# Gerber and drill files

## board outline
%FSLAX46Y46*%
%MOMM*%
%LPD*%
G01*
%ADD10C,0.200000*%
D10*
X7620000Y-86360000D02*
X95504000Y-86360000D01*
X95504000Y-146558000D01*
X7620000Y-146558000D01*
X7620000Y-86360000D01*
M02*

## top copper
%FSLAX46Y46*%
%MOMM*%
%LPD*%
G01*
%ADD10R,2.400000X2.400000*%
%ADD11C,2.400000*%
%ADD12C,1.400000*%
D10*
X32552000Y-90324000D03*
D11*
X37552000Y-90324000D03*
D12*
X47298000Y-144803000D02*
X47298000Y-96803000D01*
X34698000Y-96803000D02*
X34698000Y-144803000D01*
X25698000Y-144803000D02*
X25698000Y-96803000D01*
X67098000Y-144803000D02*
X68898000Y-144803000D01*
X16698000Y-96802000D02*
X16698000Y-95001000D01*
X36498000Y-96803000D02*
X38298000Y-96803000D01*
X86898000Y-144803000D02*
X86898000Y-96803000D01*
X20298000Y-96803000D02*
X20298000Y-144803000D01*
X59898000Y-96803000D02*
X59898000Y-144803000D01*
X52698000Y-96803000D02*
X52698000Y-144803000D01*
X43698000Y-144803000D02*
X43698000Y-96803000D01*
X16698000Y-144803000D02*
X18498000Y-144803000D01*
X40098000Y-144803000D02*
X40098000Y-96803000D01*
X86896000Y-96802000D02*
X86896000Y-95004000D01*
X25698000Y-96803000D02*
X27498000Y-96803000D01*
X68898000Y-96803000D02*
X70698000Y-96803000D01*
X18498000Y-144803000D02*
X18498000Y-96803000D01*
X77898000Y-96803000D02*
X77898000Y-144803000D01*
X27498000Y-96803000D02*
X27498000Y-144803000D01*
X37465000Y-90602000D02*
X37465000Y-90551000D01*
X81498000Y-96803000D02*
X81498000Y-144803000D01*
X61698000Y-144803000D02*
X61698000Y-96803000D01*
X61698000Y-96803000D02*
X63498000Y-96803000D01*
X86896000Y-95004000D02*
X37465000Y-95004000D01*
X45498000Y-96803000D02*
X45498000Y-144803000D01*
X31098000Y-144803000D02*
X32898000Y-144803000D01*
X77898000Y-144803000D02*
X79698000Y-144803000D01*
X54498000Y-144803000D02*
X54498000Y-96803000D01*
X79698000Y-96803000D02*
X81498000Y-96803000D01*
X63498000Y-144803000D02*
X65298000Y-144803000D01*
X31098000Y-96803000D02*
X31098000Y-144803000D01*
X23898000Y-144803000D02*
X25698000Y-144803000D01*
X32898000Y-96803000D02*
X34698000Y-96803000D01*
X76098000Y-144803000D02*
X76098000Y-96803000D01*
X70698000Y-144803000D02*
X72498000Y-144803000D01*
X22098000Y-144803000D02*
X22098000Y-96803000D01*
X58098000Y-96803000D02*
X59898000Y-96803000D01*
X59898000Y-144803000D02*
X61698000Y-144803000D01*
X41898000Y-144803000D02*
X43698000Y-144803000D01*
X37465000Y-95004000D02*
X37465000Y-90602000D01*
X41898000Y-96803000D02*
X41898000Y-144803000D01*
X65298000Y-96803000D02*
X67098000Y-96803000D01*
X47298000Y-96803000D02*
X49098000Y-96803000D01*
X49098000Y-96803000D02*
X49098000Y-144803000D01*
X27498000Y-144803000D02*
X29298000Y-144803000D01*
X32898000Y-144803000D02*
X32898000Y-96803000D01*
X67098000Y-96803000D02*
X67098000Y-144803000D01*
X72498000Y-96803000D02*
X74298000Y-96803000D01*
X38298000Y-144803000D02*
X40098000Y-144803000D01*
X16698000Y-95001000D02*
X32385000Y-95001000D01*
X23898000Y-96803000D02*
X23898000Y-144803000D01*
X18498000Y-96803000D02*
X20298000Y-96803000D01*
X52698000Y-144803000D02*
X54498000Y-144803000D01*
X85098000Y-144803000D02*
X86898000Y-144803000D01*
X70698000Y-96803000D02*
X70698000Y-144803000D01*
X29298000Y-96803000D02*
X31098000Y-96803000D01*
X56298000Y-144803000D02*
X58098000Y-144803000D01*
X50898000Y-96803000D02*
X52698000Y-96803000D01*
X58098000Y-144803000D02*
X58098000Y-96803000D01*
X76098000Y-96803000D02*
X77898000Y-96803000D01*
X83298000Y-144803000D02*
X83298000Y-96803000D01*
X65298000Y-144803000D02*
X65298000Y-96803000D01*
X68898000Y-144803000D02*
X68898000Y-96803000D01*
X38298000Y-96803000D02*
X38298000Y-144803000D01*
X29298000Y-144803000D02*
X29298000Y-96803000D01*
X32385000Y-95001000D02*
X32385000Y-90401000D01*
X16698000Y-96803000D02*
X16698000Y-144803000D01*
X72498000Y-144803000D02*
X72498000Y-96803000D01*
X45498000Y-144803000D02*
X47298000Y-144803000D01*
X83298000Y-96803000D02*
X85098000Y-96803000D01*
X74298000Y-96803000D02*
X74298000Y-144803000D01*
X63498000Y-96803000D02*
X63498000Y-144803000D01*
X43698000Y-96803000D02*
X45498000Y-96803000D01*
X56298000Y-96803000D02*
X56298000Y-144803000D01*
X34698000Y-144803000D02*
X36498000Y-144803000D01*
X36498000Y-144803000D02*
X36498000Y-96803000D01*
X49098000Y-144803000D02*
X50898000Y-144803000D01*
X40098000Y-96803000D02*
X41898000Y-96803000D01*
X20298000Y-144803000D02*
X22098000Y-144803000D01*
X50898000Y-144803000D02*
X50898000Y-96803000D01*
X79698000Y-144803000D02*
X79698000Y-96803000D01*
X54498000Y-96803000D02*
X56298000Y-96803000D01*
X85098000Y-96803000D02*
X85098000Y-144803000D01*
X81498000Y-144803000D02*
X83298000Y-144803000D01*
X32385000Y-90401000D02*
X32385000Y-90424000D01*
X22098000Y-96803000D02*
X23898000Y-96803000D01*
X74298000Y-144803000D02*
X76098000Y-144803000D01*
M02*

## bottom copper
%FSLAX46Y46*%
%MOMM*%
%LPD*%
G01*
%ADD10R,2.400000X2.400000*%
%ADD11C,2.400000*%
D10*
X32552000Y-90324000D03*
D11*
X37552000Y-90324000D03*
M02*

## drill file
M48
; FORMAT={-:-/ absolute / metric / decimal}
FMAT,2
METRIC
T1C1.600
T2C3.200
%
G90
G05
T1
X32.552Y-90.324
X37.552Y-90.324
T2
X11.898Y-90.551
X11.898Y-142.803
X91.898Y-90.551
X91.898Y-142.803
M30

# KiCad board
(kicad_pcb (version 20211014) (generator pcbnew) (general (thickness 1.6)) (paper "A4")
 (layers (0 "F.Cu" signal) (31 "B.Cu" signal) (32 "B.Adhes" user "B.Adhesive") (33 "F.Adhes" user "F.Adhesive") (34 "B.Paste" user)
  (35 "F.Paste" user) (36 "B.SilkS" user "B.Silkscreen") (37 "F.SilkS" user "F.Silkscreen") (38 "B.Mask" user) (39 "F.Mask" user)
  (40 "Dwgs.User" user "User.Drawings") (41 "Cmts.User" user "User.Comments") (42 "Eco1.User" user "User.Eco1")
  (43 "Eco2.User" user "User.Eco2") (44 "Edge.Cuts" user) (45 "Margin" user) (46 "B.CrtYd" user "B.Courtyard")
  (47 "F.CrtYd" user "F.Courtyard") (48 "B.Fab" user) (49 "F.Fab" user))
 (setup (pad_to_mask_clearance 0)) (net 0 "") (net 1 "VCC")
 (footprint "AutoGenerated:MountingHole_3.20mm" (layer "F.Cu") (at 91.898 142.803)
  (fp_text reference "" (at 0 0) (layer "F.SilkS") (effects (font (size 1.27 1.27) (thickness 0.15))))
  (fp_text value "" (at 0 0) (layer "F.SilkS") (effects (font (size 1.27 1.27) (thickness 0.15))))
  (pad "" np_thru_hole circle locked (at 0 0) (size 3.2 3.2) (drill 3.2) (layers *.Cu *.Mask)))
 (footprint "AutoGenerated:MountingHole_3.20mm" (layer "F.Cu") (at 11.898 90.551)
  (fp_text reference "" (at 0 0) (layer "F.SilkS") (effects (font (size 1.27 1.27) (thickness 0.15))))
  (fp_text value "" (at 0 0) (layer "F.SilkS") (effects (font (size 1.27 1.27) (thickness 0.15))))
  (pad "" np_thru_hole circle locked (at 0 0) (size 3.2 3.2) (drill 3.2) (layers *.Cu *.Mask)))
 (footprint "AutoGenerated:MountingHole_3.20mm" (layer "F.Cu") (at 91.898 90.551)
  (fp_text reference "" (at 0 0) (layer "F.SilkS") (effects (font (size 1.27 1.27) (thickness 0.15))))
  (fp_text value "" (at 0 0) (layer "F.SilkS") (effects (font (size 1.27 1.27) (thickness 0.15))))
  (pad "" np_thru_hole circle locked (at 0 0) (size 3.2 3.2) (drill 3.2) (layers *.Cu *.Mask)))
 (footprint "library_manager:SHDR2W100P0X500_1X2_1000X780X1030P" (layer "F.Cu") (at 32.552 90.324)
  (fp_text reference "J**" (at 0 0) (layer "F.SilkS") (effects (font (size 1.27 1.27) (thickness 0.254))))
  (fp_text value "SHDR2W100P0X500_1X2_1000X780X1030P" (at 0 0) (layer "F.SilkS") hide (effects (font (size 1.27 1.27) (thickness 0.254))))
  (pad "1" thru_hole rect locked (at 0 0) (size 2.4 2.4) (drill 1.6) (layers *.Cu *.Mask))
  (pad "2" thru_hole circle locked (at 5 0) (size 2.4 2.4) (drill 1.6) (layers *.Cu *.Mask)))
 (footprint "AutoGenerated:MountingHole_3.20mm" (layer "F.Cu") (at 11.898 142.803)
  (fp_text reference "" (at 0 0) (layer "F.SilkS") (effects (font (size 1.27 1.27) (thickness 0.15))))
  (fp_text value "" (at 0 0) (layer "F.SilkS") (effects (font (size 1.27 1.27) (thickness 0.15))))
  (pad "" np_thru_hole circle locked (at 0 0) (size 3.2 3.2) (drill 3.2) (layers *.Cu *.Mask)))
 (gr_rect (start 7.62 86.36) (end 95.504 146.558) (layer "Edge.Cuts") (width 0.2) (fill none))
 (segment (start 47.298 144.803) (end 47.298 96.803) (width 1.4) (layer "F.Cu") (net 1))
 (segment (start 34.698 96.803) (end 34.698 144.803) (width 1.4) (layer "F.Cu") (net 1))
 (segment (start 25.698 144.803) (end 25.698 96.803) (width 1.4) (layer "F.Cu") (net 1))
 (segment (start 67.098 144.803) (end 68.898 144.803) (width 1.4) (layer "F.Cu") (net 1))
 (segment (start 16.698 96.802) (end 16.698 95.001) (width 1.4) (layer "F.Cu") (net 1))
 (segment (start 36.498 96.803) (end 38.298 96.803) (width 1.4) (layer "F.Cu") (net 1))
 (segment (start 86.898 144.803) (end 86.898 96.803) (width 1.4) (layer "F.Cu") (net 1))
 (segment (start 20.298 96.803) (end 20.298 144.803) (width 1.4) (layer "F.Cu") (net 1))
 (segment (start 59.898 96.803) (end 59.898 144.803) (width 1.4) (layer "F.Cu") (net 1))
 (segment (start 52.698 96.803) (end 52.698 144.803) (width 1.4) (layer "F.Cu") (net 1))
 (segment (start 43.698 144.803) (end 43.698 96.803) (width 1.4) (layer "F.Cu") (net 1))
 (segment (start 16.698 144.803) (end 18.498 144.803) (width 1.4) (layer "F.Cu") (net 1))
 (segment (start 40.098 144.803) (end 40.098 96.803) (width 1.4) (layer "F.Cu") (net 1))
 (segment (start 86.896 96.802) (end 86.896 95.004) (width 1.4) (layer "F.Cu") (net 1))
 (segment (start 25.698 96.803) (end 27.498 96.803) (width 1.4) (layer "F.Cu") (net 1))
 (segment (start 68.898 96.803) (end 70.698 96.803) (width 1.4) (layer "F.Cu") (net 1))
 (segment (start 18.498 144.803) (end 18.498 96.803) (width 1.4) (layer "F.Cu") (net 1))
 (segment (start 77.898 96.803) (end 77.898 144.803) (width 1.4) (layer "F.Cu") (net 1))
 (segment (start 27.498 96.803) (end 27.498 144.803) (width 1.4) (layer "F.Cu") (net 1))
 (segment (start 37.465 90.602) (end 37.465 90.551) (width 1.4) (layer "F.Cu") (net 1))
 (segment (start 81.498 96.803) (end 81.498 144.803) (width 1.4) (layer "F.Cu") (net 1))
 (segment (start 61.698 144.803) (end 61.698 96.803) (width 1.4) (layer "F.Cu") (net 1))
 (segment (start 61.698 96.803) (end 63.498 96.803) (width 1.4) (layer "F.Cu") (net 1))
 (segment (start 86.896 95.004) (end 37.465 95.004) (width 1.4) (layer "F.Cu") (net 1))
 (segment (start 45.498 96.803) (end 45.498 144.803) (width 1.4) (layer "F.Cu") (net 1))
 (segment (start 31.098 144.803) (end 32.898 144.803) (width 1.4) (layer "F.Cu") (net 1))
 (segment (start 77.898 144.803) (end 79.698 144.803) (width 1.4) (layer "F.Cu") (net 1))
 (segment (start 54.498 144.803) (end 54.498 96.803) (width 1.4) (layer "F.Cu") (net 1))
 (segment (start 79.698 96.803) (end 81.498 96.803) (width 1.4) (layer "F.Cu") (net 1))
 (segment (start 63.498 144.803) (end 65.298 144.803) (width 1.4) (layer "F.Cu") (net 1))
 (segment (start 31.098 96.803) (end 31.098 144.803) (width 1.4) (layer "F.Cu") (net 1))
 (segment (start 23.898 144.803) (end 25.698 144.803) (width 1.4) (layer "F.Cu") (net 1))
 (segment (start 32.898 96.803) (end 34.698 96.803) (width 1.4) (layer "F.Cu") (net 1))
 (segment (start 76.098 144.803) (end 76.098 96.803) (width 1.4) (layer "F.Cu") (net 1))
 (segment (start 70.698 144.803) (end 72.498 144.803) (width 1.4) (layer "F.Cu") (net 1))
 (segment (start 22.098 144.803) (end 22.098 96.803) (width 1.4) (layer "F.Cu") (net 1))
 (segment (start 58.098 96.803) (end 59.898 96.803) (width 1.4) (layer "F.Cu") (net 1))
 (segment (start 59.898 144.803) (end 61.698 144.803) (width 1.4) (layer "F.Cu") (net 1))
 (segment (start 41.898 144.803) (end 43.698 144.803) (width 1.4) (layer "F.Cu") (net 1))
 (segment (start 37.465 95.004) (end 37.465 90.602) (width 1.4) (layer "F.Cu") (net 1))
 (segment (start 41.898 96.803) (end 41.898 144.803) (width 1.4) (layer "F.Cu") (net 1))
 (segment (start 65.298 96.803) (end 67.098 96.803) (width 1.4) (layer "F.Cu") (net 1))
 (segment (start 47.298 96.803) (end 49.098 96.803) (width 1.4) (layer "F.Cu") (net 1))
 (segment (start 49.098 96.803) (end 49.098 144.803) (width 1.4) (layer "F.Cu") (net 1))
 (segment (start 27.498 144.803) (end 29.298 144.803) (width 1.4) (layer "F.Cu") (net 1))
 (segment (start 32.898 144.803) (end 32.898 96.803) (width 1.4) (layer "F.Cu") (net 1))
 (segment (start 67.098 96.803) (end 67.098 144.803) (width 1.4) (layer "F.Cu") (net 1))
 (segment (start 72.498 96.803) (end 74.298 96.803) (width 1.4) (layer "F.Cu") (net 1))
 (segment (start 38.298 144.803) (end 40.098 144.803) (width 1.4) (layer "F.Cu") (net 1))
 (segment (start 16.698 95.001) (end 32.385 95.001) (width 1.4) (layer "F.Cu") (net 1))
 (segment (start 23.898 96.803) (end 23.898 144.803) (width 1.4) (layer "F.Cu") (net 1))
 (segment (start 18.498 96.803) (end 20.298 96.803) (width 1.4) (layer "F.Cu") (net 1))
 (segment (start 52.698 144.803) (end 54.498 144.803) (width 1.4) (layer "F.Cu") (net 1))
 (segment (start 85.098 144.803) (end 86.898 144.803) (width 1.4) (layer "F.Cu") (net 1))
 (segment (start 70.698 96.803) (end 70.698 144.803) (width 1.4) (layer "F.Cu") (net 1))
 (segment (start 29.298 96.803) (end 31.098 96.803) (width 1.4) (layer "F.Cu") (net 1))
 (segment (start 56.298 144.803) (end 58.098 144.803) (width 1.4) (layer "F.Cu") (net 1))
 (segment (start 50.898 96.803) (end 52.698 96.803) (width 1.4) (layer "F.Cu") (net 1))
 (segment (start 58.098 144.803) (end 58.098 96.803) (width 1.4) (layer "F.Cu") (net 1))
 (segment (start 76.098 96.803) (end 77.898 96.803) (width 1.4) (layer "F.Cu") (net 1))
 (segment (start 83.298 144.803) (end 83.298 96.803) (width 1.4) (layer "F.Cu") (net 1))
 (segment (start 65.298 144.803) (end 65.298 96.803) (width 1.4) (layer "F.Cu") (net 1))
 (segment (start 68.898 144.803) (end 68.898 96.803) (width 1.4) (layer "F.Cu") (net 1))
 (segment (start 38.298 96.803) (end 38.298 144.803) (width 1.4) (layer "F.Cu") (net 1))
 (segment (start 29.298 144.803) (end 29.298 96.803) (width 1.4) (layer "F.Cu") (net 1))
 (segment (start 32.385 95.001) (end 32.385 90.401) (width 1.4) (layer "F.Cu") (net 1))
 (segment (start 16.698 96.803) (end 16.698 144.803) (width 1.4) (layer "F.Cu") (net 1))
 (segment (start 72.498 144.803) (end 72.498 96.803) (width 1.4) (layer "F.Cu") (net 1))
 (segment (start 45.498 144.803) (end 47.298 144.803) (width 1.4) (layer "F.Cu") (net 1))
 (segment (start 83.298 96.803) (end 85.098 96.803) (width 1.4) (layer "F.Cu") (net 1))
 (segment (start 74.298 96.803) (end 74.298 144.803) (width 1.4) (layer "F.Cu") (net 1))
 (segment (start 63.498 96.803) (end 63.498 144.803) (width 1.4) (layer "F.Cu") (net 1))
 (segment (start 43.698 96.803) (end 45.498 96.803) (width 1.4) (layer "F.Cu") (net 1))
 (segment (start 56.298 96.803) (end 56.298 144.803) (width 1.4) (layer "F.Cu") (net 1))
 (segment (start 34.698 144.803) (end 36.498 144.803) (width 1.4) (layer "F.Cu") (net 1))
 (segment (start 36.498 144.803) (end 36.498 96.803) (width 1.4) (layer "F.Cu") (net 1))
 (segment (start 49.098 144.803) (end 50.898 144.803) (width 1.4) (layer "F.Cu") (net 1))
 (segment (start 40.098 96.803) (end 41.898 96.803) (width 1.4) (layer "F.Cu") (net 1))
 (segment (start 20.298 144.803) (end 22.098 144.803) (width 1.4) (layer "F.Cu") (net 1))
 (segment (start 50.898 144.803) (end 50.898 96.803) (width 1.4) (layer "F.Cu") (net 1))
 (segment (start 79.698 144.803) (end 79.698 96.803) (width 1.4) (layer "F.Cu") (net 1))
 (segment (start 54.498 96.803) (end 56.298 96.803) (width 1.4) (layer "F.Cu") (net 1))
 (segment (start 85.098 96.803) (end 85.098 144.803) (width 1.4) (layer "F.Cu") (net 1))
 (segment (start 81.498 144.803) (end 83.298 144.803) (width 1.4) (layer "F.Cu") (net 1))
 (segment (start 32.385 90.401) (end 32.385 90.424) (width 1.4) (layer "F.Cu") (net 1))
 (segment (start 22.098 96.803) (end 23.898 96.803) (width 1.4) (layer "F.Cu") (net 1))
 (segment (start 74.298 144.803) (end 76.098 144.803) (width 1.4) (layer "F.Cu") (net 1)))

